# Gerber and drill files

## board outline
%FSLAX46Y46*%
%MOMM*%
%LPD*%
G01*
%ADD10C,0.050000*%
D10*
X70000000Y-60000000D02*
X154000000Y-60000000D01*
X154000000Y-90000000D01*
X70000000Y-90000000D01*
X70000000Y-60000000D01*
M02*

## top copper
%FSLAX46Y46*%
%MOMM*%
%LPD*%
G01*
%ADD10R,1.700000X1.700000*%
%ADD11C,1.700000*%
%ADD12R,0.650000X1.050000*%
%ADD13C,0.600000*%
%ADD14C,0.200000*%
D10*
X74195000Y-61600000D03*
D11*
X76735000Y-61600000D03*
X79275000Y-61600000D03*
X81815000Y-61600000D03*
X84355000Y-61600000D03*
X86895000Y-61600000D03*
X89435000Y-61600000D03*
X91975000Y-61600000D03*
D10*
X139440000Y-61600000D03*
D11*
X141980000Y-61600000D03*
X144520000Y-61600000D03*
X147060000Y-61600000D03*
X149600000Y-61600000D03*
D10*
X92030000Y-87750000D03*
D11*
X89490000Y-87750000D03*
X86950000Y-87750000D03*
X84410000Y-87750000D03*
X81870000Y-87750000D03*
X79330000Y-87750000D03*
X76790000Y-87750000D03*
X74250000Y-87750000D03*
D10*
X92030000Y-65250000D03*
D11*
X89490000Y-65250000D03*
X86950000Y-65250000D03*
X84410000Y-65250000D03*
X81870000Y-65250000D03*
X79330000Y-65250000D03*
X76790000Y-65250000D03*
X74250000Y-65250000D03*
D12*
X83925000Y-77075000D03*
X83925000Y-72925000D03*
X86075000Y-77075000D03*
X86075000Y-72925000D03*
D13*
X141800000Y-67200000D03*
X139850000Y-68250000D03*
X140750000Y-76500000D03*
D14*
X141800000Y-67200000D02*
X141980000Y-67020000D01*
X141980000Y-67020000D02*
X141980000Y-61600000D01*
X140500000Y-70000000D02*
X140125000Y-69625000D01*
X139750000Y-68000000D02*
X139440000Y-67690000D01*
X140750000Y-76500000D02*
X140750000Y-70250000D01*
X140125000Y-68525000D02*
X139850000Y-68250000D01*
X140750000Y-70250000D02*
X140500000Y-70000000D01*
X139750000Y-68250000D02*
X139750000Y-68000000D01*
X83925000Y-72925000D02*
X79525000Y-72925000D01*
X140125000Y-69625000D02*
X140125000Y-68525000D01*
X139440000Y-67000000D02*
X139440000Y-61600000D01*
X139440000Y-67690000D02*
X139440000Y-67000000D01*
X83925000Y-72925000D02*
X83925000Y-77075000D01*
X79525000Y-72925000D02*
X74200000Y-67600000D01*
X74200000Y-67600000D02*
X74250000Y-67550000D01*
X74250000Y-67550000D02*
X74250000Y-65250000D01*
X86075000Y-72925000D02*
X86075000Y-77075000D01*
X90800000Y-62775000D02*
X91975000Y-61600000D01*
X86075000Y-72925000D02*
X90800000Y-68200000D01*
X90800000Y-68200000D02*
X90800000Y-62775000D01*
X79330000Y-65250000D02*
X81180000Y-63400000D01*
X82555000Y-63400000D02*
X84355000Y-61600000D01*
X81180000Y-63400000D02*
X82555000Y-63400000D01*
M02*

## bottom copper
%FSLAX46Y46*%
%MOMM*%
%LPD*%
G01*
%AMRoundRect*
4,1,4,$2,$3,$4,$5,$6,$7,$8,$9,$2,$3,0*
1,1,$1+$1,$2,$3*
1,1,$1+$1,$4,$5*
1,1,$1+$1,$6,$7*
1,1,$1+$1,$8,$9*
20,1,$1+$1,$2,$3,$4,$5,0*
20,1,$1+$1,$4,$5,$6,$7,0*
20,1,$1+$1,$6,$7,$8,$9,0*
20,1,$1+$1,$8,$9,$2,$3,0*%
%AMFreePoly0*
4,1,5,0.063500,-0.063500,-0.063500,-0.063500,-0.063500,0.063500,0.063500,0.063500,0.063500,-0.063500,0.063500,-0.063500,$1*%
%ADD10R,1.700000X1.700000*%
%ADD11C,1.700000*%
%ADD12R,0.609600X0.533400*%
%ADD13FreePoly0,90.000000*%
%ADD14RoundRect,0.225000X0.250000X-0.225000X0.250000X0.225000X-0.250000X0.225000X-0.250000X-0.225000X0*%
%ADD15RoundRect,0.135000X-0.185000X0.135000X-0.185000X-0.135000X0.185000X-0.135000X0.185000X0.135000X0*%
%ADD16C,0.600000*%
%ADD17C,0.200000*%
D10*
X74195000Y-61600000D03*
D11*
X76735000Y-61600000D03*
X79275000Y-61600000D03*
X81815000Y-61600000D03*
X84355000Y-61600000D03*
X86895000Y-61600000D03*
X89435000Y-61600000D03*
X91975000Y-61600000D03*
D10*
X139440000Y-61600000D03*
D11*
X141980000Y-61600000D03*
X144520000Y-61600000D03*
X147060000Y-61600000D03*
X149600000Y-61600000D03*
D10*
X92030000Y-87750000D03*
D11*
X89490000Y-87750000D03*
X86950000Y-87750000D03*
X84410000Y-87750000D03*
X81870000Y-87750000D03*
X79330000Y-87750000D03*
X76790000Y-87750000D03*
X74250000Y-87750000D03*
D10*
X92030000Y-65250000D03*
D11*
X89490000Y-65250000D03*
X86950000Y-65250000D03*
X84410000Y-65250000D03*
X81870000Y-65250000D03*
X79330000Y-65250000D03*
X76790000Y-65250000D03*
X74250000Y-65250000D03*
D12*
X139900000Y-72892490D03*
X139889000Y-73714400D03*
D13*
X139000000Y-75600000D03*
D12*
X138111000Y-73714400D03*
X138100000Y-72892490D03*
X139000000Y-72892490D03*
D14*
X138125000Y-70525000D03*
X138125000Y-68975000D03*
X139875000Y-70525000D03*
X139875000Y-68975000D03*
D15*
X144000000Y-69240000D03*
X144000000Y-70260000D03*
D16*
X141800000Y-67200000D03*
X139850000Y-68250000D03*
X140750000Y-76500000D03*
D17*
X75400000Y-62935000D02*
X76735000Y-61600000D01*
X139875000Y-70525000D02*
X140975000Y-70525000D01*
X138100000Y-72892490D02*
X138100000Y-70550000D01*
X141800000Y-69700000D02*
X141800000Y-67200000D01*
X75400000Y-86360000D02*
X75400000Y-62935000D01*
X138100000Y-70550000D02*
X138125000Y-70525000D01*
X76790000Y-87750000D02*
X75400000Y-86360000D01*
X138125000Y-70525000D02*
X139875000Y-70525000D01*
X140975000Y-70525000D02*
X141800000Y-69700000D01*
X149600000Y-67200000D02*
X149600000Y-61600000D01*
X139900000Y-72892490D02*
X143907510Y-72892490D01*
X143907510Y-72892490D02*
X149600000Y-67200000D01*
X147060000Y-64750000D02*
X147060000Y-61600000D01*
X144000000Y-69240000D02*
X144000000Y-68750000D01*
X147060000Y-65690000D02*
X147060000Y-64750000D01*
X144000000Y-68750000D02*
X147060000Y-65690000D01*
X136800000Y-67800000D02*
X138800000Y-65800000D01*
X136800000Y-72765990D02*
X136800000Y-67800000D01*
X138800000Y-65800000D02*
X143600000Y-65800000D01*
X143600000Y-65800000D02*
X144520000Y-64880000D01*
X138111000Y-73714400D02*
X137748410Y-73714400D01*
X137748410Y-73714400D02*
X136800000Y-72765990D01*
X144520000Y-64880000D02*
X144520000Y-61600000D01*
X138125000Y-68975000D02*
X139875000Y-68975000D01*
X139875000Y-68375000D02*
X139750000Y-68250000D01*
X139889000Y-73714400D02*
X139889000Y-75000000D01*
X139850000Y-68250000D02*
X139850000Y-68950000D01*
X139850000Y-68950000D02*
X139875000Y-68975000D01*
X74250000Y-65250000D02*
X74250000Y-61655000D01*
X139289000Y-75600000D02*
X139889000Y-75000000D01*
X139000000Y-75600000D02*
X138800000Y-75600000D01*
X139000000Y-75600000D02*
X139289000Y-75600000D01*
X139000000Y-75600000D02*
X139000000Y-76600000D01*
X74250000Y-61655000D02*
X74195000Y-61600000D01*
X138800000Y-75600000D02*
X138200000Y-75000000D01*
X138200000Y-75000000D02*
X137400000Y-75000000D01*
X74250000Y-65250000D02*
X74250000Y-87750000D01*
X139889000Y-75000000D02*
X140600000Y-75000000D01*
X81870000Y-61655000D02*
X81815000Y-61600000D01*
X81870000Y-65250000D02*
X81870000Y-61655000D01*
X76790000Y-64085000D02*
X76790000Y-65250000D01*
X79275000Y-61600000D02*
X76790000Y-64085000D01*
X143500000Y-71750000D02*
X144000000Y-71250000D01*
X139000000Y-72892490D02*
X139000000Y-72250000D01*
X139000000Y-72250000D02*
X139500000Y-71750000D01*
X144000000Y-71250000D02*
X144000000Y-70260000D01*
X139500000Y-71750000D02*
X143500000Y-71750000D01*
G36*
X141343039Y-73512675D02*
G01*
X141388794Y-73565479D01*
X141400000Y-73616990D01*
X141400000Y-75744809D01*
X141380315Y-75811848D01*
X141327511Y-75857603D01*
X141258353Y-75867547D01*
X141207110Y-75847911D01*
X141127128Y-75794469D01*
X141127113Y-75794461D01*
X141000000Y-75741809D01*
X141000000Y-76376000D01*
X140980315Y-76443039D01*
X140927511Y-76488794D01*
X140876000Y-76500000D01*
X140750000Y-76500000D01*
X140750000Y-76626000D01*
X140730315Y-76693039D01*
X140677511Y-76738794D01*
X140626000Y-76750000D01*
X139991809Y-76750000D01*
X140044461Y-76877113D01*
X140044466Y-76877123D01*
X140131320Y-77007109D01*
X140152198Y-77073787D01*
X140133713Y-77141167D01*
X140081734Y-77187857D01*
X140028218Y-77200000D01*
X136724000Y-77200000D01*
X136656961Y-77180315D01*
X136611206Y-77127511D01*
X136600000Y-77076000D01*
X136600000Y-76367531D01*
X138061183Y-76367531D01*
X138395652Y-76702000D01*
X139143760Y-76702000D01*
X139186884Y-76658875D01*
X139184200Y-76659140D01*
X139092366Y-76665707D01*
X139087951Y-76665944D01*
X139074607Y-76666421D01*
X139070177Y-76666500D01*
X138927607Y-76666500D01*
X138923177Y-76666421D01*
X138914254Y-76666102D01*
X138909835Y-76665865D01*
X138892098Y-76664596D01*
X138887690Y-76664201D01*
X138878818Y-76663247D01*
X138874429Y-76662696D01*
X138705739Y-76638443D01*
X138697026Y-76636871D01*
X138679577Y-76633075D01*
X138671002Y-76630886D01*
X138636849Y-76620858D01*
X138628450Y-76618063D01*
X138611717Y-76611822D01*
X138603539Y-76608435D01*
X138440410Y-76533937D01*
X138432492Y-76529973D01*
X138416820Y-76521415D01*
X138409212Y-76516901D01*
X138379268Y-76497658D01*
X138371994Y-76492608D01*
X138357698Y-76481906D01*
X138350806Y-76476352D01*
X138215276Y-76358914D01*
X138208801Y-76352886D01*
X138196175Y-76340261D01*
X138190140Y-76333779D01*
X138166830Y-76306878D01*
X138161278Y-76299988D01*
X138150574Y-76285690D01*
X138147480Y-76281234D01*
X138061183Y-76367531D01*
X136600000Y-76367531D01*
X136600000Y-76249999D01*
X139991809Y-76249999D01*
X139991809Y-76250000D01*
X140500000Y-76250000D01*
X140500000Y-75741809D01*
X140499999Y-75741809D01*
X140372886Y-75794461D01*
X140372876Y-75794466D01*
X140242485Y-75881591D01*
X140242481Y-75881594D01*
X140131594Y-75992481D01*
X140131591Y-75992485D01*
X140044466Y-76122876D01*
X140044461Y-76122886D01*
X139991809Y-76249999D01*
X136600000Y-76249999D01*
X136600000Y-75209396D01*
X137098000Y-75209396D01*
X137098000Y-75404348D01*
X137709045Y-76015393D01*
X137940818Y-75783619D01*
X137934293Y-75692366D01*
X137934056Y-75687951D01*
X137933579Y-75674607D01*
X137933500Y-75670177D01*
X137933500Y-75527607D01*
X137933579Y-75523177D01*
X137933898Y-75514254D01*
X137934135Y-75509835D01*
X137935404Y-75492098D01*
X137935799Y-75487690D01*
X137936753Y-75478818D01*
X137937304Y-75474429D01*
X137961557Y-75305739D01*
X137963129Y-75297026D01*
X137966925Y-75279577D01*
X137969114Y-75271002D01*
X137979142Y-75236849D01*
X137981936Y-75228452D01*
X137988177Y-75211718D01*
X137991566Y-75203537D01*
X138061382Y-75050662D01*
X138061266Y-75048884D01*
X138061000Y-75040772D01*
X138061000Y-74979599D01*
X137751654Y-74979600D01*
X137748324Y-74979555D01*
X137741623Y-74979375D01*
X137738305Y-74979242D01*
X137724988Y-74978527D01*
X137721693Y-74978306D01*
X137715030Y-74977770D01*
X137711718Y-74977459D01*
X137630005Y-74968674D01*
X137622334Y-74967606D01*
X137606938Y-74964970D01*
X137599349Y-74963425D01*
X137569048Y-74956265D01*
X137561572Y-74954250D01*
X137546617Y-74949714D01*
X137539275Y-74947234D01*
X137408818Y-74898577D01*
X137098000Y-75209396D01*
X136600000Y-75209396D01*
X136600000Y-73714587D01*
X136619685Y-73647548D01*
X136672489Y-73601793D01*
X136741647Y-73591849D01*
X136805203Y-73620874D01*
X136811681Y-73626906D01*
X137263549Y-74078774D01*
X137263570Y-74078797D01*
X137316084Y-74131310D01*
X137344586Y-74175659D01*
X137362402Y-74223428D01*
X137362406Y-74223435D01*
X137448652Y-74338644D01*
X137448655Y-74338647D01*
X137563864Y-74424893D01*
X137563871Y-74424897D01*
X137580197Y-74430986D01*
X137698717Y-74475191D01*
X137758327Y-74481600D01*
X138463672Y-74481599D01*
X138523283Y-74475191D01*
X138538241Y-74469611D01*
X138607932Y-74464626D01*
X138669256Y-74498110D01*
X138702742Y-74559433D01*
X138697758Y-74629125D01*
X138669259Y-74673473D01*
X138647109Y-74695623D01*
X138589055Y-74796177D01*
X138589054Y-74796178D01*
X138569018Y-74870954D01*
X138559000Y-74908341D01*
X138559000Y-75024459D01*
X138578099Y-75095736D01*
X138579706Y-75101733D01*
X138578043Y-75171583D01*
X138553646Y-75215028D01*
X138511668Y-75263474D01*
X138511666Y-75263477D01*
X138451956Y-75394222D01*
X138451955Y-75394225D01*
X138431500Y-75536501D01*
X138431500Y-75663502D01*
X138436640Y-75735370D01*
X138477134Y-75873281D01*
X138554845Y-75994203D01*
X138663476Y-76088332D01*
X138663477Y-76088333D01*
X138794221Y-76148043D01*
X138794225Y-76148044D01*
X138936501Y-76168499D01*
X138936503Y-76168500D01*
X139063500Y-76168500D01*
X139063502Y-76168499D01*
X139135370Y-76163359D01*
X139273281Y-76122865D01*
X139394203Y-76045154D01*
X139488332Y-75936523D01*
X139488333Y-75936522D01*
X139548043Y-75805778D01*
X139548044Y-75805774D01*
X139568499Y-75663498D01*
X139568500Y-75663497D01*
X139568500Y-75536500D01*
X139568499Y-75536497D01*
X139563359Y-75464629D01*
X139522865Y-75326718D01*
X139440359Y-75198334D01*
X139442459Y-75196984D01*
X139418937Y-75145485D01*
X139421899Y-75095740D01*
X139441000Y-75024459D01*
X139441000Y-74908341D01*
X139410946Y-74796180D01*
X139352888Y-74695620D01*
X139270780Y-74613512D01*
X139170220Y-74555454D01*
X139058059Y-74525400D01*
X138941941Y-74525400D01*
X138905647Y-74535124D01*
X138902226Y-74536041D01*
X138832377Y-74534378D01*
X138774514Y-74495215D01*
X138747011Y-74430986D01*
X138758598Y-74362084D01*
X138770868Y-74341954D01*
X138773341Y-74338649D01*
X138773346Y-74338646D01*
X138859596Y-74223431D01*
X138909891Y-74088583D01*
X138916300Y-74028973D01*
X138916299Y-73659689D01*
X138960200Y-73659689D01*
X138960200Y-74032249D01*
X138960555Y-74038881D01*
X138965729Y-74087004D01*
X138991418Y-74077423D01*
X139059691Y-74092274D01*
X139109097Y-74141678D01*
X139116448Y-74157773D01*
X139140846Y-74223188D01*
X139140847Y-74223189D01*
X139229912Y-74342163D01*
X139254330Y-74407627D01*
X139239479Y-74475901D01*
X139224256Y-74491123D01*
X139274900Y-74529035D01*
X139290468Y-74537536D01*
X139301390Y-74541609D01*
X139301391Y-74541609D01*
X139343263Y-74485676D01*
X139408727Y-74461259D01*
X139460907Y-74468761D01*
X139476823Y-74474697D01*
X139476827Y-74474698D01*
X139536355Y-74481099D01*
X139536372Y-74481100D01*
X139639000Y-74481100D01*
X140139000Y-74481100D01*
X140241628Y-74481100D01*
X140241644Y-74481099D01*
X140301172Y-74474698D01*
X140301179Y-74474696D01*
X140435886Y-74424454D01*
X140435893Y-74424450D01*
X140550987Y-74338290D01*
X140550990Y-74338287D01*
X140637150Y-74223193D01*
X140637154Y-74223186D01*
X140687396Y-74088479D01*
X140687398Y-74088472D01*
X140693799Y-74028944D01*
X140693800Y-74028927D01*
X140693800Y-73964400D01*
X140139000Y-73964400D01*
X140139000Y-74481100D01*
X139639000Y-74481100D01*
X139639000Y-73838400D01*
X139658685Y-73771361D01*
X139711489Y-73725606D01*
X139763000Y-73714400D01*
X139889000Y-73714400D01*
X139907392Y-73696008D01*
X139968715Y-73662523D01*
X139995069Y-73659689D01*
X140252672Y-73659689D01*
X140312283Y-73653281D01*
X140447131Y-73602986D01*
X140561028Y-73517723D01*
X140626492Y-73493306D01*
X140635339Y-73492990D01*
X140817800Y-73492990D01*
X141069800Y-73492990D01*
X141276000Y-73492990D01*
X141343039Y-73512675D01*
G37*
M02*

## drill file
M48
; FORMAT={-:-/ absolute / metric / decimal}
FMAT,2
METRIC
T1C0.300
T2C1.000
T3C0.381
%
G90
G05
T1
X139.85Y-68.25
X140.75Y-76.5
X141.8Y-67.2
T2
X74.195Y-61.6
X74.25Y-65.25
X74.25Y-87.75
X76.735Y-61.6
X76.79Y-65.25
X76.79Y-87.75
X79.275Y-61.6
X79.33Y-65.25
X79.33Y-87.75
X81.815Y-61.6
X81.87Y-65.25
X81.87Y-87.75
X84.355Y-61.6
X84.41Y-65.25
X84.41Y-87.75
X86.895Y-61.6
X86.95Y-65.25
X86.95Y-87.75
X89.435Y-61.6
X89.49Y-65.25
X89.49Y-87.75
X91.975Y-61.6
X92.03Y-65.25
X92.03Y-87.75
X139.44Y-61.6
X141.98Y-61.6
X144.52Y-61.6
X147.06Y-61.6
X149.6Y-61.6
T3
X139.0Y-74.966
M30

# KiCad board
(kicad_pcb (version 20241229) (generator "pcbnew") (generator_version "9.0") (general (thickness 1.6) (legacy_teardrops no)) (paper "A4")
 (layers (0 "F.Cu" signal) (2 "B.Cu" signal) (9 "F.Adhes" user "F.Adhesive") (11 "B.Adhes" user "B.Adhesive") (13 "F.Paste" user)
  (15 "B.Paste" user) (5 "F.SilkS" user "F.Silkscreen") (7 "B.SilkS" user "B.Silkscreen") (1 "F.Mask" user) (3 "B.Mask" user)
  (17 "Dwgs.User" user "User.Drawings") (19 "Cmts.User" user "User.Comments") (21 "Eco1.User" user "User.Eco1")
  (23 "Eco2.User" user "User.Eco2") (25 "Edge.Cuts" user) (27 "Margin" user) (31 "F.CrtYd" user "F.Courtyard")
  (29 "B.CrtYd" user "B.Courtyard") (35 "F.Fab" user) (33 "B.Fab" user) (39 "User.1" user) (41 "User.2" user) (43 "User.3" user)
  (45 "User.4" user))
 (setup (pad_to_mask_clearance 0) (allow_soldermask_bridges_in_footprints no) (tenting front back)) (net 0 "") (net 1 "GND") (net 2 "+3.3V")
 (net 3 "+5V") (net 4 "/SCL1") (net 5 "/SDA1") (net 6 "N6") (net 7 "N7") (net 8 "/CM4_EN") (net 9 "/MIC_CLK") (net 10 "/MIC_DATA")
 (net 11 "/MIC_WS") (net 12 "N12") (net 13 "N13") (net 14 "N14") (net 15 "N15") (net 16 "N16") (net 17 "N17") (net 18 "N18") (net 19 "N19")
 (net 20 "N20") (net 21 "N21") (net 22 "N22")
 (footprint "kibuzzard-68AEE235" (layer "F.Cu") (at 78.05 69.05 -90)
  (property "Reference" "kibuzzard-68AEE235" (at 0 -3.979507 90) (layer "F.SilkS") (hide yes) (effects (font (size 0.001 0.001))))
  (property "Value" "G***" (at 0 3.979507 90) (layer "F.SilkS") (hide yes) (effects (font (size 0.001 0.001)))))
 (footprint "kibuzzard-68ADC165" (layer "F.Cu") (at 147.25 75)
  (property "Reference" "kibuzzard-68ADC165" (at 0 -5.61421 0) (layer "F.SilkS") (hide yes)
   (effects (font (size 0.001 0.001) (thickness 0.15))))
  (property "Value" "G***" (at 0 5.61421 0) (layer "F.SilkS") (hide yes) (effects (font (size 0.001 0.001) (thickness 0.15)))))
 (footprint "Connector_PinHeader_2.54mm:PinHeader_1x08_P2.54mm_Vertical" (layer "F.Cu") (at 74.195 61.6 90)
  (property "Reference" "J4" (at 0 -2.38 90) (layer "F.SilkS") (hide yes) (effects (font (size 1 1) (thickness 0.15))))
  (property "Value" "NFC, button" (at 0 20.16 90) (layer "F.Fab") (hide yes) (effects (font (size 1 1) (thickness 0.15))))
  (pad "1" thru_hole rect (at 0 0 90) (size 1.7 1.7) (drill 1) (layers "*.Cu" "*.Mask") (remove_unused_layers no) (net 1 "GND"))
  (pad "2" thru_hole circle (at 0 2.54 90) (size 1.7 1.7) (drill 1) (layers "*.Cu" "*.Mask") (remove_unused_layers no) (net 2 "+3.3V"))
  (pad "3" thru_hole circle (at 0 5.08 90) (size 1.7 1.7) (drill 1) (layers "*.Cu" "*.Mask") (remove_unused_layers no) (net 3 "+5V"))
  (pad "4" thru_hole circle (at 0 7.62 90) (size 1.7 1.7) (drill 1) (layers "*.Cu" "*.Mask") (remove_unused_layers no) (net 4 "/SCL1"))
  (pad "5" thru_hole circle (at 0 10.16 90) (size 1.7 1.7) (drill 1) (layers "*.Cu" "*.Mask") (remove_unused_layers no) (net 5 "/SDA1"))
  (pad "6" thru_hole circle (at 0 12.7 90) (size 1.7 1.7) (drill 1) (layers "*.Cu" "*.Mask") (remove_unused_layers no) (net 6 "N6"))
  (pad "7" thru_hole circle (at 0 15.24 90) (size 1.7 1.7) (drill 1) (layers "*.Cu" "*.Mask") (remove_unused_layers no) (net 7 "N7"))
  (pad "8" thru_hole circle (at 0 17.78 90) (size 1.7 1.7) (drill 1) (layers "*.Cu" "*.Mask") (remove_unused_layers no) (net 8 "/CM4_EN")))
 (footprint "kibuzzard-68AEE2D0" (layer "F.Cu") (at 83.15 69 -90)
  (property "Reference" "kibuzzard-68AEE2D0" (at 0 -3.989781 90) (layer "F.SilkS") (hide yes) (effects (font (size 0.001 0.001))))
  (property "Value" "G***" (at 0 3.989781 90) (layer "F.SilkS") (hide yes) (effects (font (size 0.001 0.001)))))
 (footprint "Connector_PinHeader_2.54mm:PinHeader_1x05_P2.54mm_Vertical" (layer "F.Cu") (at 139.44 61.6 90)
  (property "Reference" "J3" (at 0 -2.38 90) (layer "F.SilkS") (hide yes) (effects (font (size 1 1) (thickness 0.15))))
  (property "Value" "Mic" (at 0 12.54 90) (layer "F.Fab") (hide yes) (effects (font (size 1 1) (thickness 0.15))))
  (pad "1" thru_hole rect (at 0 0 90) (size 1.7 1.7) (drill 1) (layers "*.Cu" "*.Mask") (remove_unused_layers no) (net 1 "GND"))
  (pad "2" thru_hole circle (at 0 2.54 90) (size 1.7 1.7) (drill 1) (layers "*.Cu" "*.Mask") (remove_unused_layers no) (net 2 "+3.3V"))
  (pad "3" thru_hole circle (at 0 5.08 90) (size 1.7 1.7) (drill 1) (layers "*.Cu" "*.Mask") (remove_unused_layers no) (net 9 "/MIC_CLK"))
  (pad "4" thru_hole circle (at 0 7.62 90) (size 1.7 1.7) (drill 1) (layers "*.Cu" "*.Mask") (remove_unused_layers no) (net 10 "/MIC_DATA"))
  (pad "5" thru_hole circle (at 0 10.16 90) (size 1.7 1.7) (drill 1) (layers "*.Cu" "*.Mask") (remove_unused_layers no) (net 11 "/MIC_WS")))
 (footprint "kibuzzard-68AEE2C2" (layer "F.Cu") (at 80.6 69 -90)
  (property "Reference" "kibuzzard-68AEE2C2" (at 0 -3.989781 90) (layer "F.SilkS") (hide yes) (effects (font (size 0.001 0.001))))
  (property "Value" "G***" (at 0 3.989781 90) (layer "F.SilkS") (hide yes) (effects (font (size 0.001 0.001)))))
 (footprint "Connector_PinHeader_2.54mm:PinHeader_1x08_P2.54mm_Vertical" (layer "F.Cu") (at 92.03 87.75 -90)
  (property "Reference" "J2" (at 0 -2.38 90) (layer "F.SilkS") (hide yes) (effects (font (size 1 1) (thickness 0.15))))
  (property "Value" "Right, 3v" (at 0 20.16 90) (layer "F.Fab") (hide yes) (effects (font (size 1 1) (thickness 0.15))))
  (pad "1" thru_hole rect (at 0 0 270) (size 1.7 1.7) (drill 1) (layers "*.Cu" "*.Mask") (remove_unused_layers no) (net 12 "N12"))
  (pad "2" thru_hole circle (at 0 2.54 270) (size 1.7 1.7) (drill 1) (layers "*.Cu" "*.Mask") (remove_unused_layers no) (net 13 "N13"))
  (pad "3" thru_hole circle (at 0 5.08 270) (size 1.7 1.7) (drill 1) (layers "*.Cu" "*.Mask") (remove_unused_layers no) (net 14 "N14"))
  (pad "4" thru_hole circle (at 0 7.62 270) (size 1.7 1.7) (drill 1) (layers "*.Cu" "*.Mask") (remove_unused_layers no) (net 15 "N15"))
  (pad "5" thru_hole circle (at 0 10.16 270) (size 1.7 1.7) (drill 1) (layers "*.Cu" "*.Mask") (remove_unused_layers no) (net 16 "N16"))
  (pad "6" thru_hole circle (at 0 12.7 270) (size 1.7 1.7) (drill 1) (layers "*.Cu" "*.Mask") (remove_unused_layers no) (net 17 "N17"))
  (pad "7" thru_hole circle (at 0 15.24 270) (size 1.7 1.7) (drill 1) (layers "*.Cu" "*.Mask") (remove_unused_layers no) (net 2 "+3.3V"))
  (pad "8" thru_hole circle (at 0 17.78 270) (size 1.7 1.7) (drill 1) (layers "*.Cu" "*.Mask") (remove_unused_layers no) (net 1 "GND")))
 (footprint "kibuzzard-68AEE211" (layer "F.Cu") (at 72.969178 69.071804 -90)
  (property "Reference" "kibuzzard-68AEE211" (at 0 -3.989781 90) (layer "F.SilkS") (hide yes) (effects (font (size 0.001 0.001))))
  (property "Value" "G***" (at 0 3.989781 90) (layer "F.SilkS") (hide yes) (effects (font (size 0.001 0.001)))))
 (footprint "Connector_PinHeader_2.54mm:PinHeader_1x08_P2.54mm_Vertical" (layer "F.Cu") (at 92.03 65.25 -90)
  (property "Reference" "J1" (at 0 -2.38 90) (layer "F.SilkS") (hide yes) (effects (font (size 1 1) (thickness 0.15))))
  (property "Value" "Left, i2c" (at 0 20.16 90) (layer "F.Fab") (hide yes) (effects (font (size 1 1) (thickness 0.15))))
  (pad "1" thru_hole rect (at 0 0 270) (size 1.7 1.7) (drill 1) (layers "*.Cu" "*.Mask") (remove_unused_layers no) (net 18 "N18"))
  (pad "2" thru_hole circle (at 0 2.54 270) (size 1.7 1.7) (drill 1) (layers "*.Cu" "*.Mask") (remove_unused_layers no) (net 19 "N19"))
  (pad "3" thru_hole circle (at 0 5.08 270) (size 1.7 1.7) (drill 1) (layers "*.Cu" "*.Mask") (remove_unused_layers no) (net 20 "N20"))
  (pad "4" thru_hole circle (at 0 7.62 270) (size 1.7 1.7) (drill 1) (layers "*.Cu" "*.Mask") (remove_unused_layers no) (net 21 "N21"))
  (pad "5" thru_hole circle (at 0 10.16 270) (size 1.7 1.7) (drill 1) (layers "*.Cu" "*.Mask") (remove_unused_layers no) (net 4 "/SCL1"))
  (pad "6" thru_hole circle (at 0 12.7 270) (size 1.7 1.7) (drill 1) (layers "*.Cu" "*.Mask") (remove_unused_layers no) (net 5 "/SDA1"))
  (pad "7" thru_hole circle (at 0 15.24 270) (size 1.7 1.7) (drill 1) (layers "*.Cu" "*.Mask") (remove_unused_layers no) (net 3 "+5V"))
  (pad "8" thru_hole circle (at 0 17.78 270) (size 1.7 1.7) (drill 1) (layers "*.Cu" "*.Mask") (remove_unused_layers no) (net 1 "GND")))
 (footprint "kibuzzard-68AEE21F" (layer "F.Cu") (at 75.55 70.1 -90)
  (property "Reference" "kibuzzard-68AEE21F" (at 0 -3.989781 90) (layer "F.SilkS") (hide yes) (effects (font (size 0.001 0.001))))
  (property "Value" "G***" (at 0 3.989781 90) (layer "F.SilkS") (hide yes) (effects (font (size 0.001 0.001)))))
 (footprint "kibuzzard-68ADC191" (layer "F.Cu") (at 113.6 75)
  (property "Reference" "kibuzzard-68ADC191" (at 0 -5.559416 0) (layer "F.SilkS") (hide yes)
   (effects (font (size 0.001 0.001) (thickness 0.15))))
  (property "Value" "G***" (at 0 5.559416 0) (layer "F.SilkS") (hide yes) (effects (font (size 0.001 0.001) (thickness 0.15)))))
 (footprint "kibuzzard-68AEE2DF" (layer "F.Cu") (at 90.8 70.55 -90)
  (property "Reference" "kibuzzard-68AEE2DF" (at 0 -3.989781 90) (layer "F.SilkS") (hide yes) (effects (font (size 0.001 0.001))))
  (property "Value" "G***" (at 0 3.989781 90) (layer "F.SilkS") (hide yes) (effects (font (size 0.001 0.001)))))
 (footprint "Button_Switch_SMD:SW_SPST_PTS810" (layer "F.Cu") (at 85 75 90)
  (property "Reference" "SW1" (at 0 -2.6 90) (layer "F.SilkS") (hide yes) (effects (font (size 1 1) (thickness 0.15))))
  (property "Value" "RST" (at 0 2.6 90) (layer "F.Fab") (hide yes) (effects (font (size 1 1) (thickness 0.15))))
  (pad "1" smd rect (at -2.075 -1.075 90) (size 1.05 0.65) (layers "F.Cu" "F.Mask" "F.Paste") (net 1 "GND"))
  (pad "1" smd rect (at 2.075 -1.075 90) (size 1.05 0.65) (layers "F.Cu" "F.Mask" "F.Paste") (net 1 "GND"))
  (pad "2" smd rect (at -2.075 1.075 90) (size 1.05 0.65) (layers "F.Cu" "F.Mask" "F.Paste") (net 8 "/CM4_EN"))
  (pad "2" smd rect (at 2.075 1.075 90) (size 1.05 0.65) (layers "F.Cu" "F.Mask" "F.Paste") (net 8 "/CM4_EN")))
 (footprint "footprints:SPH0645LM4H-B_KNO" (layer "B.Cu") (at 139 74.203 90)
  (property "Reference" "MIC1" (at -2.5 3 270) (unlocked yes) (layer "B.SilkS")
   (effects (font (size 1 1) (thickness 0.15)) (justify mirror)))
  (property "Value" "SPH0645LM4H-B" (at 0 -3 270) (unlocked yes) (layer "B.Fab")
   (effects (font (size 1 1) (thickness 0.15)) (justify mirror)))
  (pad "" np_thru_hole circle (at -0.7634 0 90) (size 0.381 0.381) (drill 0.381) (layers))
  (pad "1" smd rect (at 1.31051 0.9 90) (size 0.5334 0.6096) (layers "B.Cu" "B.Mask" "B.Paste") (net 11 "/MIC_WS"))
  (pad "2" smd rect (at 0.4886 0.889 90) (size 0.5334 0.6096) (layers "B.Cu" "B.Mask" "B.Paste") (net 1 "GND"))
  (pad "3" smd custom (at -1.397 0 90) (size 0.127 0.127) (layers "B.Cu" "B.Mask" "B.Paste") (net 1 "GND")
   (options (clearance outline) (anchor rect)) (primitives))
  (pad "4" smd rect (at 0.4886 -0.889 90) (size 0.5334 0.6096) (layers "B.Cu" "B.Mask" "B.Paste") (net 9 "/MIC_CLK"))
  (pad "5" smd rect (at 1.31051 -0.9 90) (size 0.5334 0.6096) (layers "B.Cu" "B.Mask" "B.Paste") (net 2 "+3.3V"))
  (pad "6" smd rect (at 1.31051 0 90) (size 0.5334 0.6096) (layers "B.Cu" "B.Mask" "B.Paste") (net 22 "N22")))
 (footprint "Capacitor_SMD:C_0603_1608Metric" (layer "B.Cu") (at 138.125 69.75 90)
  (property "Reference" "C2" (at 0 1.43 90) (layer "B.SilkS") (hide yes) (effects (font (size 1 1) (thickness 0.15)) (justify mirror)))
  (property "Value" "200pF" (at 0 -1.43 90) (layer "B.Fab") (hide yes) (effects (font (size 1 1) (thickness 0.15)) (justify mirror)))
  (pad "1" smd roundrect (at -0.775 0 90) (size 0.9 0.95) (layers "B.Cu" "B.Mask" "B.Paste") (roundrect_rratio 0.25) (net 2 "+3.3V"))
  (pad "2" smd roundrect (at 0.775 0 90) (size 0.9 0.95) (layers "B.Cu" "B.Mask" "B.Paste") (roundrect_rratio 0.25) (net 1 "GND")))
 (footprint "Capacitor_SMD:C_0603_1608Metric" (layer "B.Cu") (at 139.875 69.75 90)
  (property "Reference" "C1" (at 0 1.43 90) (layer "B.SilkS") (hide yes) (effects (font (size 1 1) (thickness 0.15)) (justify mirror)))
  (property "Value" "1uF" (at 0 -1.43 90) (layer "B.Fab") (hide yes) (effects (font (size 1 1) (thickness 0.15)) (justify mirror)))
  (pad "1" smd roundrect (at -0.775 0 90) (size 0.9 0.95) (layers "B.Cu" "B.Mask" "B.Paste") (roundrect_rratio 0.25) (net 2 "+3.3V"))
  (pad "2" smd roundrect (at 0.775 0 90) (size 0.9 0.95) (layers "B.Cu" "B.Mask" "B.Paste") (roundrect_rratio 0.25) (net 1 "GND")))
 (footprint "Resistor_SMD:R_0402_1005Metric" (layer "B.Cu") (at 144 69.75 -90)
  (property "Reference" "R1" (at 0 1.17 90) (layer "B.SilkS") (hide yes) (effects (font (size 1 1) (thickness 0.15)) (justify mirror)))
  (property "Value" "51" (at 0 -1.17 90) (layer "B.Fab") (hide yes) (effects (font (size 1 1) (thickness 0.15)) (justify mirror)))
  (pad "1" smd roundrect (at -0.51 0 270) (size 0.54 0.64) (layers "B.Cu" "B.Mask" "B.Paste") (roundrect_rratio 0.25) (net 10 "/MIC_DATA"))
  (pad "2" smd roundrect (at 0.51 0 270) (size 0.54 0.64) (layers "B.Cu" "B.Mask" "B.Paste") (roundrect_rratio 0.25) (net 22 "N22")))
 (gr_rect (start 70 60) (end 154 90) (stroke (width 0.05) (type default)) (fill no) (layer "Edge.Cuts"))
 (segment (start 141.8 67.2) (end 141.98 67.02) (width 0.2) (layer "F.Cu") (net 2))
 (segment (start 141.98 67.02) (end 141.98 61.6) (width 0.2) (layer "F.Cu") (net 2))
 (via (at 141.8 67.2) (size 0.6) (drill 0.3) (layers "F.Cu" "B.Cu") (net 2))
 (segment (start 75.4 62.935) (end 76.735 61.6) (width 0.2) (layer "B.Cu") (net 2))
 (segment (start 139.875 70.525) (end 140.975 70.525) (width 0.2) (layer "B.Cu") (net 2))
 (segment (start 138.1 72.89249) (end 138.1 70.55) (width 0.2) (layer "B.Cu") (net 2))
 (segment (start 141.8 69.7) (end 141.8 67.2) (width 0.2) (layer "B.Cu") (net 2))
 (segment (start 75.4 86.36) (end 75.4 62.935) (width 0.2) (layer "B.Cu") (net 2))
 (segment (start 138.1 70.55) (end 138.125 70.525) (width 0.2) (layer "B.Cu") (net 2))
 (segment (start 76.79 87.75) (end 75.4 86.36) (width 0.2) (layer "B.Cu") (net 2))
 (segment (start 138.125 70.525) (end 139.875 70.525) (width 0.2) (layer "B.Cu") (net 2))
 (segment (start 140.975 70.525) (end 141.8 69.7) (width 0.2) (layer "B.Cu") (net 2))
 (segment (start 149.6 67.2) (end 149.6 61.6) (width 0.2) (layer "B.Cu") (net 11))
 (segment (start 139.9 72.89249) (end 143.90751 72.89249) (width 0.2) (layer "B.Cu") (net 11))
 (segment (start 143.90751 72.89249) (end 149.6 67.2) (width 0.2) (layer "B.Cu") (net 11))
 (segment (start 147.06 64.75) (end 147.06 61.6) (width 0.2) (layer "B.Cu") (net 10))
 (segment (start 144 69.24) (end 144 68.75) (width 0.2) (layer "B.Cu") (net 10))
 (segment (start 147.06 65.69) (end 147.06 64.75) (width 0.2) (layer "B.Cu") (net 10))
 (segment (start 144 68.75) (end 147.06 65.69) (width 0.2) (layer "B.Cu") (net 10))
 (segment (start 136.8 67.8) (end 138.8 65.8) (width 0.2) (layer "B.Cu") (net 9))
 (segment (start 136.8 72.76599) (end 136.8 67.8) (width 0.2) (layer "B.Cu") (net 9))
 (segment (start 138.8 65.8) (end 143.6 65.8) (width 0.2) (layer "B.Cu") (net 9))
 (segment (start 143.6 65.8) (end 144.52 64.88) (width 0.2) (layer "B.Cu") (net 9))
 (segment (start 138.111 73.7144) (end 137.74841 73.7144) (width 0.2) (layer "B.Cu") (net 9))
 (segment (start 137.74841 73.7144) (end 136.8 72.76599) (width 0.2) (layer "B.Cu") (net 9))
 (segment (start 144.52 64.88) (end 144.52 61.6) (width 0.2) (layer "B.Cu") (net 9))
 (segment (start 140.5 70) (end 140.125 69.625) (width 0.2) (layer "F.Cu") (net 1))
 (segment (start 139.75 68) (end 139.44 67.69) (width 0.2) (layer "F.Cu") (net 1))
 (segment (start 140.75 76.5) (end 140.75 70.25) (width 0.2) (layer "F.Cu") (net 1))
 (segment (start 140.125 68.525) (end 139.85 68.25) (width 0.2) (layer "F.Cu") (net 1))
 (segment (start 140.75 70.25) (end 140.5 70) (width 0.2) (layer "F.Cu") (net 1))
 (segment (start 139.75 68.25) (end 139.75 68) (width 0.2) (layer "F.Cu") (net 1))
 (segment (start 83.925 72.925) (end 79.525 72.925) (width 0.2) (layer "F.Cu") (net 1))
 (segment (start 140.125 69.625) (end 140.125 68.525) (width 0.2) (layer "F.Cu") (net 1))
 (segment (start 139.44 67) (end 139.44 61.6) (width 0.2) (layer "F.Cu") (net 1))
 (segment (start 139.44 67.69) (end 139.44 67) (width 0.2) (layer "F.Cu") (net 1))
 (segment (start 83.925 72.925) (end 83.925 77.075) (width 0.2) (layer "F.Cu") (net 1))
 (segment (start 79.525 72.925) (end 74.2 67.6) (width 0.2) (layer "F.Cu") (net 1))
 (segment (start 74.2 67.6) (end 74.25 67.55) (width 0.2) (layer "F.Cu") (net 1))
 (segment (start 74.25 67.55) (end 74.25 65.25) (width 0.2) (layer "F.Cu") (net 1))
 (via (at 139.85 68.25) (size 0.6) (drill 0.3) (layers "F.Cu" "B.Cu") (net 1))
 (via (at 140.75 76.5) (size 0.6) (drill 0.3) (layers "F.Cu" "B.Cu") (free yes) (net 1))
 (segment (start 138.125 68.975) (end 139.875 68.975) (width 0.2) (layer "B.Cu") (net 1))
 (segment (start 139.875 68.375) (end 139.75 68.25) (width 0.2) (layer "B.Cu") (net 1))
 (segment (start 139.889 73.7144) (end 139.889 75) (width 0.2) (layer "B.Cu") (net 1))
 (segment (start 139.85 68.25) (end 139.85 68.95) (width 0.2) (layer "B.Cu") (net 1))
 (segment (start 139.85 68.95) (end 139.875 68.975) (width 0.2) (layer "B.Cu") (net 1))
 (segment (start 74.25 65.25) (end 74.25 61.655) (width 0.2) (layer "B.Cu") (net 1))
 (segment (start 139.289 75.6) (end 139.889 75) (width 0.2) (layer "B.Cu") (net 1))
 (segment (start 139 75.6) (end 138.8 75.6) (width 0.2) (layer "B.Cu") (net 1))
 (segment (start 139 75.6) (end 139.289 75.6) (width 0.2) (layer "B.Cu") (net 1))
 (segment (start 139 75.6) (end 139 76.6) (width 0.2) (layer "B.Cu") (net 1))
 (segment (start 74.25 61.655) (end 74.195 61.6) (width 0.2) (layer "B.Cu") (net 1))
 (segment (start 138.8 75.6) (end 138.2 75) (width 0.2) (layer "B.Cu") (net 1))
 (segment (start 138.2 75) (end 137.4 75) (width 0.2) (layer "B.Cu") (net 1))
 (segment (start 74.25 65.25) (end 74.25 87.75) (width 0.2) (layer "B.Cu") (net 1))
 (segment (start 139.889 75) (end 140.6 75) (width 0.2) (layer "B.Cu") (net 1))
 (segment (start 86.075 72.925) (end 86.075 77.075) (width 0.2) (layer "F.Cu") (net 8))
 (segment (start 90.8 62.775) (end 91.975 61.6) (width 0.2) (layer "F.Cu") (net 8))
 (segment (start 86.075 72.925) (end 90.8 68.2) (width 0.2) (layer "F.Cu") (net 8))
 (segment (start 90.8 68.2) (end 90.8 62.775) (width 0.2) (layer "F.Cu") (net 8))
 (segment (start 79.33 65.25) (end 81.18 63.4) (width 0.2) (layer "F.Cu") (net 5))
 (segment (start 82.555 63.4) (end 84.355 61.6) (width 0.2) (layer "F.Cu") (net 5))
 (segment (start 81.18 63.4) (end 82.555 63.4) (width 0.2) (layer "F.Cu") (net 5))
 (segment (start 81.87 61.655) (end 81.815 61.6) (width 0.2) (layer "B.Cu") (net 4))
 (segment (start 81.87 65.25) (end 81.87 61.655) (width 0.2) (layer "B.Cu") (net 4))
 (segment (start 76.79 64.085) (end 76.79 65.25) (width 0.2) (layer "B.Cu") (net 3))
 (segment (start 79.275 61.6) (end 76.79 64.085) (width 0.2) (layer "B.Cu") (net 3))
 (segment (start 143.5 71.75) (end 144 71.25) (width 0.2) (layer "B.Cu") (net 22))
 (segment (start 139 72.89249) (end 139 72.25) (width 0.2) (layer "B.Cu") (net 22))
 (segment (start 139 72.25) (end 139.5 71.75) (width 0.2) (layer "B.Cu") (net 22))
 (segment (start 144 71.25) (end 144 70.26) (width 0.2) (layer "B.Cu") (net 22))
 (segment (start 139.5 71.75) (end 143.5 71.75) (width 0.2) (layer "B.Cu") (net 22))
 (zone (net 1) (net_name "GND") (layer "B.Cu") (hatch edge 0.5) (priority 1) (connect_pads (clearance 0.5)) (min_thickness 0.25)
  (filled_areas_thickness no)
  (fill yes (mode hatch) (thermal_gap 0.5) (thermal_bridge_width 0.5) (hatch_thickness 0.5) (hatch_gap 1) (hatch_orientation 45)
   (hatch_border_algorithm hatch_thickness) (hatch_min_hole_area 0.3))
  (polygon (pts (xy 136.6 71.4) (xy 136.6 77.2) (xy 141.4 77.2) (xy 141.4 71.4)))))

